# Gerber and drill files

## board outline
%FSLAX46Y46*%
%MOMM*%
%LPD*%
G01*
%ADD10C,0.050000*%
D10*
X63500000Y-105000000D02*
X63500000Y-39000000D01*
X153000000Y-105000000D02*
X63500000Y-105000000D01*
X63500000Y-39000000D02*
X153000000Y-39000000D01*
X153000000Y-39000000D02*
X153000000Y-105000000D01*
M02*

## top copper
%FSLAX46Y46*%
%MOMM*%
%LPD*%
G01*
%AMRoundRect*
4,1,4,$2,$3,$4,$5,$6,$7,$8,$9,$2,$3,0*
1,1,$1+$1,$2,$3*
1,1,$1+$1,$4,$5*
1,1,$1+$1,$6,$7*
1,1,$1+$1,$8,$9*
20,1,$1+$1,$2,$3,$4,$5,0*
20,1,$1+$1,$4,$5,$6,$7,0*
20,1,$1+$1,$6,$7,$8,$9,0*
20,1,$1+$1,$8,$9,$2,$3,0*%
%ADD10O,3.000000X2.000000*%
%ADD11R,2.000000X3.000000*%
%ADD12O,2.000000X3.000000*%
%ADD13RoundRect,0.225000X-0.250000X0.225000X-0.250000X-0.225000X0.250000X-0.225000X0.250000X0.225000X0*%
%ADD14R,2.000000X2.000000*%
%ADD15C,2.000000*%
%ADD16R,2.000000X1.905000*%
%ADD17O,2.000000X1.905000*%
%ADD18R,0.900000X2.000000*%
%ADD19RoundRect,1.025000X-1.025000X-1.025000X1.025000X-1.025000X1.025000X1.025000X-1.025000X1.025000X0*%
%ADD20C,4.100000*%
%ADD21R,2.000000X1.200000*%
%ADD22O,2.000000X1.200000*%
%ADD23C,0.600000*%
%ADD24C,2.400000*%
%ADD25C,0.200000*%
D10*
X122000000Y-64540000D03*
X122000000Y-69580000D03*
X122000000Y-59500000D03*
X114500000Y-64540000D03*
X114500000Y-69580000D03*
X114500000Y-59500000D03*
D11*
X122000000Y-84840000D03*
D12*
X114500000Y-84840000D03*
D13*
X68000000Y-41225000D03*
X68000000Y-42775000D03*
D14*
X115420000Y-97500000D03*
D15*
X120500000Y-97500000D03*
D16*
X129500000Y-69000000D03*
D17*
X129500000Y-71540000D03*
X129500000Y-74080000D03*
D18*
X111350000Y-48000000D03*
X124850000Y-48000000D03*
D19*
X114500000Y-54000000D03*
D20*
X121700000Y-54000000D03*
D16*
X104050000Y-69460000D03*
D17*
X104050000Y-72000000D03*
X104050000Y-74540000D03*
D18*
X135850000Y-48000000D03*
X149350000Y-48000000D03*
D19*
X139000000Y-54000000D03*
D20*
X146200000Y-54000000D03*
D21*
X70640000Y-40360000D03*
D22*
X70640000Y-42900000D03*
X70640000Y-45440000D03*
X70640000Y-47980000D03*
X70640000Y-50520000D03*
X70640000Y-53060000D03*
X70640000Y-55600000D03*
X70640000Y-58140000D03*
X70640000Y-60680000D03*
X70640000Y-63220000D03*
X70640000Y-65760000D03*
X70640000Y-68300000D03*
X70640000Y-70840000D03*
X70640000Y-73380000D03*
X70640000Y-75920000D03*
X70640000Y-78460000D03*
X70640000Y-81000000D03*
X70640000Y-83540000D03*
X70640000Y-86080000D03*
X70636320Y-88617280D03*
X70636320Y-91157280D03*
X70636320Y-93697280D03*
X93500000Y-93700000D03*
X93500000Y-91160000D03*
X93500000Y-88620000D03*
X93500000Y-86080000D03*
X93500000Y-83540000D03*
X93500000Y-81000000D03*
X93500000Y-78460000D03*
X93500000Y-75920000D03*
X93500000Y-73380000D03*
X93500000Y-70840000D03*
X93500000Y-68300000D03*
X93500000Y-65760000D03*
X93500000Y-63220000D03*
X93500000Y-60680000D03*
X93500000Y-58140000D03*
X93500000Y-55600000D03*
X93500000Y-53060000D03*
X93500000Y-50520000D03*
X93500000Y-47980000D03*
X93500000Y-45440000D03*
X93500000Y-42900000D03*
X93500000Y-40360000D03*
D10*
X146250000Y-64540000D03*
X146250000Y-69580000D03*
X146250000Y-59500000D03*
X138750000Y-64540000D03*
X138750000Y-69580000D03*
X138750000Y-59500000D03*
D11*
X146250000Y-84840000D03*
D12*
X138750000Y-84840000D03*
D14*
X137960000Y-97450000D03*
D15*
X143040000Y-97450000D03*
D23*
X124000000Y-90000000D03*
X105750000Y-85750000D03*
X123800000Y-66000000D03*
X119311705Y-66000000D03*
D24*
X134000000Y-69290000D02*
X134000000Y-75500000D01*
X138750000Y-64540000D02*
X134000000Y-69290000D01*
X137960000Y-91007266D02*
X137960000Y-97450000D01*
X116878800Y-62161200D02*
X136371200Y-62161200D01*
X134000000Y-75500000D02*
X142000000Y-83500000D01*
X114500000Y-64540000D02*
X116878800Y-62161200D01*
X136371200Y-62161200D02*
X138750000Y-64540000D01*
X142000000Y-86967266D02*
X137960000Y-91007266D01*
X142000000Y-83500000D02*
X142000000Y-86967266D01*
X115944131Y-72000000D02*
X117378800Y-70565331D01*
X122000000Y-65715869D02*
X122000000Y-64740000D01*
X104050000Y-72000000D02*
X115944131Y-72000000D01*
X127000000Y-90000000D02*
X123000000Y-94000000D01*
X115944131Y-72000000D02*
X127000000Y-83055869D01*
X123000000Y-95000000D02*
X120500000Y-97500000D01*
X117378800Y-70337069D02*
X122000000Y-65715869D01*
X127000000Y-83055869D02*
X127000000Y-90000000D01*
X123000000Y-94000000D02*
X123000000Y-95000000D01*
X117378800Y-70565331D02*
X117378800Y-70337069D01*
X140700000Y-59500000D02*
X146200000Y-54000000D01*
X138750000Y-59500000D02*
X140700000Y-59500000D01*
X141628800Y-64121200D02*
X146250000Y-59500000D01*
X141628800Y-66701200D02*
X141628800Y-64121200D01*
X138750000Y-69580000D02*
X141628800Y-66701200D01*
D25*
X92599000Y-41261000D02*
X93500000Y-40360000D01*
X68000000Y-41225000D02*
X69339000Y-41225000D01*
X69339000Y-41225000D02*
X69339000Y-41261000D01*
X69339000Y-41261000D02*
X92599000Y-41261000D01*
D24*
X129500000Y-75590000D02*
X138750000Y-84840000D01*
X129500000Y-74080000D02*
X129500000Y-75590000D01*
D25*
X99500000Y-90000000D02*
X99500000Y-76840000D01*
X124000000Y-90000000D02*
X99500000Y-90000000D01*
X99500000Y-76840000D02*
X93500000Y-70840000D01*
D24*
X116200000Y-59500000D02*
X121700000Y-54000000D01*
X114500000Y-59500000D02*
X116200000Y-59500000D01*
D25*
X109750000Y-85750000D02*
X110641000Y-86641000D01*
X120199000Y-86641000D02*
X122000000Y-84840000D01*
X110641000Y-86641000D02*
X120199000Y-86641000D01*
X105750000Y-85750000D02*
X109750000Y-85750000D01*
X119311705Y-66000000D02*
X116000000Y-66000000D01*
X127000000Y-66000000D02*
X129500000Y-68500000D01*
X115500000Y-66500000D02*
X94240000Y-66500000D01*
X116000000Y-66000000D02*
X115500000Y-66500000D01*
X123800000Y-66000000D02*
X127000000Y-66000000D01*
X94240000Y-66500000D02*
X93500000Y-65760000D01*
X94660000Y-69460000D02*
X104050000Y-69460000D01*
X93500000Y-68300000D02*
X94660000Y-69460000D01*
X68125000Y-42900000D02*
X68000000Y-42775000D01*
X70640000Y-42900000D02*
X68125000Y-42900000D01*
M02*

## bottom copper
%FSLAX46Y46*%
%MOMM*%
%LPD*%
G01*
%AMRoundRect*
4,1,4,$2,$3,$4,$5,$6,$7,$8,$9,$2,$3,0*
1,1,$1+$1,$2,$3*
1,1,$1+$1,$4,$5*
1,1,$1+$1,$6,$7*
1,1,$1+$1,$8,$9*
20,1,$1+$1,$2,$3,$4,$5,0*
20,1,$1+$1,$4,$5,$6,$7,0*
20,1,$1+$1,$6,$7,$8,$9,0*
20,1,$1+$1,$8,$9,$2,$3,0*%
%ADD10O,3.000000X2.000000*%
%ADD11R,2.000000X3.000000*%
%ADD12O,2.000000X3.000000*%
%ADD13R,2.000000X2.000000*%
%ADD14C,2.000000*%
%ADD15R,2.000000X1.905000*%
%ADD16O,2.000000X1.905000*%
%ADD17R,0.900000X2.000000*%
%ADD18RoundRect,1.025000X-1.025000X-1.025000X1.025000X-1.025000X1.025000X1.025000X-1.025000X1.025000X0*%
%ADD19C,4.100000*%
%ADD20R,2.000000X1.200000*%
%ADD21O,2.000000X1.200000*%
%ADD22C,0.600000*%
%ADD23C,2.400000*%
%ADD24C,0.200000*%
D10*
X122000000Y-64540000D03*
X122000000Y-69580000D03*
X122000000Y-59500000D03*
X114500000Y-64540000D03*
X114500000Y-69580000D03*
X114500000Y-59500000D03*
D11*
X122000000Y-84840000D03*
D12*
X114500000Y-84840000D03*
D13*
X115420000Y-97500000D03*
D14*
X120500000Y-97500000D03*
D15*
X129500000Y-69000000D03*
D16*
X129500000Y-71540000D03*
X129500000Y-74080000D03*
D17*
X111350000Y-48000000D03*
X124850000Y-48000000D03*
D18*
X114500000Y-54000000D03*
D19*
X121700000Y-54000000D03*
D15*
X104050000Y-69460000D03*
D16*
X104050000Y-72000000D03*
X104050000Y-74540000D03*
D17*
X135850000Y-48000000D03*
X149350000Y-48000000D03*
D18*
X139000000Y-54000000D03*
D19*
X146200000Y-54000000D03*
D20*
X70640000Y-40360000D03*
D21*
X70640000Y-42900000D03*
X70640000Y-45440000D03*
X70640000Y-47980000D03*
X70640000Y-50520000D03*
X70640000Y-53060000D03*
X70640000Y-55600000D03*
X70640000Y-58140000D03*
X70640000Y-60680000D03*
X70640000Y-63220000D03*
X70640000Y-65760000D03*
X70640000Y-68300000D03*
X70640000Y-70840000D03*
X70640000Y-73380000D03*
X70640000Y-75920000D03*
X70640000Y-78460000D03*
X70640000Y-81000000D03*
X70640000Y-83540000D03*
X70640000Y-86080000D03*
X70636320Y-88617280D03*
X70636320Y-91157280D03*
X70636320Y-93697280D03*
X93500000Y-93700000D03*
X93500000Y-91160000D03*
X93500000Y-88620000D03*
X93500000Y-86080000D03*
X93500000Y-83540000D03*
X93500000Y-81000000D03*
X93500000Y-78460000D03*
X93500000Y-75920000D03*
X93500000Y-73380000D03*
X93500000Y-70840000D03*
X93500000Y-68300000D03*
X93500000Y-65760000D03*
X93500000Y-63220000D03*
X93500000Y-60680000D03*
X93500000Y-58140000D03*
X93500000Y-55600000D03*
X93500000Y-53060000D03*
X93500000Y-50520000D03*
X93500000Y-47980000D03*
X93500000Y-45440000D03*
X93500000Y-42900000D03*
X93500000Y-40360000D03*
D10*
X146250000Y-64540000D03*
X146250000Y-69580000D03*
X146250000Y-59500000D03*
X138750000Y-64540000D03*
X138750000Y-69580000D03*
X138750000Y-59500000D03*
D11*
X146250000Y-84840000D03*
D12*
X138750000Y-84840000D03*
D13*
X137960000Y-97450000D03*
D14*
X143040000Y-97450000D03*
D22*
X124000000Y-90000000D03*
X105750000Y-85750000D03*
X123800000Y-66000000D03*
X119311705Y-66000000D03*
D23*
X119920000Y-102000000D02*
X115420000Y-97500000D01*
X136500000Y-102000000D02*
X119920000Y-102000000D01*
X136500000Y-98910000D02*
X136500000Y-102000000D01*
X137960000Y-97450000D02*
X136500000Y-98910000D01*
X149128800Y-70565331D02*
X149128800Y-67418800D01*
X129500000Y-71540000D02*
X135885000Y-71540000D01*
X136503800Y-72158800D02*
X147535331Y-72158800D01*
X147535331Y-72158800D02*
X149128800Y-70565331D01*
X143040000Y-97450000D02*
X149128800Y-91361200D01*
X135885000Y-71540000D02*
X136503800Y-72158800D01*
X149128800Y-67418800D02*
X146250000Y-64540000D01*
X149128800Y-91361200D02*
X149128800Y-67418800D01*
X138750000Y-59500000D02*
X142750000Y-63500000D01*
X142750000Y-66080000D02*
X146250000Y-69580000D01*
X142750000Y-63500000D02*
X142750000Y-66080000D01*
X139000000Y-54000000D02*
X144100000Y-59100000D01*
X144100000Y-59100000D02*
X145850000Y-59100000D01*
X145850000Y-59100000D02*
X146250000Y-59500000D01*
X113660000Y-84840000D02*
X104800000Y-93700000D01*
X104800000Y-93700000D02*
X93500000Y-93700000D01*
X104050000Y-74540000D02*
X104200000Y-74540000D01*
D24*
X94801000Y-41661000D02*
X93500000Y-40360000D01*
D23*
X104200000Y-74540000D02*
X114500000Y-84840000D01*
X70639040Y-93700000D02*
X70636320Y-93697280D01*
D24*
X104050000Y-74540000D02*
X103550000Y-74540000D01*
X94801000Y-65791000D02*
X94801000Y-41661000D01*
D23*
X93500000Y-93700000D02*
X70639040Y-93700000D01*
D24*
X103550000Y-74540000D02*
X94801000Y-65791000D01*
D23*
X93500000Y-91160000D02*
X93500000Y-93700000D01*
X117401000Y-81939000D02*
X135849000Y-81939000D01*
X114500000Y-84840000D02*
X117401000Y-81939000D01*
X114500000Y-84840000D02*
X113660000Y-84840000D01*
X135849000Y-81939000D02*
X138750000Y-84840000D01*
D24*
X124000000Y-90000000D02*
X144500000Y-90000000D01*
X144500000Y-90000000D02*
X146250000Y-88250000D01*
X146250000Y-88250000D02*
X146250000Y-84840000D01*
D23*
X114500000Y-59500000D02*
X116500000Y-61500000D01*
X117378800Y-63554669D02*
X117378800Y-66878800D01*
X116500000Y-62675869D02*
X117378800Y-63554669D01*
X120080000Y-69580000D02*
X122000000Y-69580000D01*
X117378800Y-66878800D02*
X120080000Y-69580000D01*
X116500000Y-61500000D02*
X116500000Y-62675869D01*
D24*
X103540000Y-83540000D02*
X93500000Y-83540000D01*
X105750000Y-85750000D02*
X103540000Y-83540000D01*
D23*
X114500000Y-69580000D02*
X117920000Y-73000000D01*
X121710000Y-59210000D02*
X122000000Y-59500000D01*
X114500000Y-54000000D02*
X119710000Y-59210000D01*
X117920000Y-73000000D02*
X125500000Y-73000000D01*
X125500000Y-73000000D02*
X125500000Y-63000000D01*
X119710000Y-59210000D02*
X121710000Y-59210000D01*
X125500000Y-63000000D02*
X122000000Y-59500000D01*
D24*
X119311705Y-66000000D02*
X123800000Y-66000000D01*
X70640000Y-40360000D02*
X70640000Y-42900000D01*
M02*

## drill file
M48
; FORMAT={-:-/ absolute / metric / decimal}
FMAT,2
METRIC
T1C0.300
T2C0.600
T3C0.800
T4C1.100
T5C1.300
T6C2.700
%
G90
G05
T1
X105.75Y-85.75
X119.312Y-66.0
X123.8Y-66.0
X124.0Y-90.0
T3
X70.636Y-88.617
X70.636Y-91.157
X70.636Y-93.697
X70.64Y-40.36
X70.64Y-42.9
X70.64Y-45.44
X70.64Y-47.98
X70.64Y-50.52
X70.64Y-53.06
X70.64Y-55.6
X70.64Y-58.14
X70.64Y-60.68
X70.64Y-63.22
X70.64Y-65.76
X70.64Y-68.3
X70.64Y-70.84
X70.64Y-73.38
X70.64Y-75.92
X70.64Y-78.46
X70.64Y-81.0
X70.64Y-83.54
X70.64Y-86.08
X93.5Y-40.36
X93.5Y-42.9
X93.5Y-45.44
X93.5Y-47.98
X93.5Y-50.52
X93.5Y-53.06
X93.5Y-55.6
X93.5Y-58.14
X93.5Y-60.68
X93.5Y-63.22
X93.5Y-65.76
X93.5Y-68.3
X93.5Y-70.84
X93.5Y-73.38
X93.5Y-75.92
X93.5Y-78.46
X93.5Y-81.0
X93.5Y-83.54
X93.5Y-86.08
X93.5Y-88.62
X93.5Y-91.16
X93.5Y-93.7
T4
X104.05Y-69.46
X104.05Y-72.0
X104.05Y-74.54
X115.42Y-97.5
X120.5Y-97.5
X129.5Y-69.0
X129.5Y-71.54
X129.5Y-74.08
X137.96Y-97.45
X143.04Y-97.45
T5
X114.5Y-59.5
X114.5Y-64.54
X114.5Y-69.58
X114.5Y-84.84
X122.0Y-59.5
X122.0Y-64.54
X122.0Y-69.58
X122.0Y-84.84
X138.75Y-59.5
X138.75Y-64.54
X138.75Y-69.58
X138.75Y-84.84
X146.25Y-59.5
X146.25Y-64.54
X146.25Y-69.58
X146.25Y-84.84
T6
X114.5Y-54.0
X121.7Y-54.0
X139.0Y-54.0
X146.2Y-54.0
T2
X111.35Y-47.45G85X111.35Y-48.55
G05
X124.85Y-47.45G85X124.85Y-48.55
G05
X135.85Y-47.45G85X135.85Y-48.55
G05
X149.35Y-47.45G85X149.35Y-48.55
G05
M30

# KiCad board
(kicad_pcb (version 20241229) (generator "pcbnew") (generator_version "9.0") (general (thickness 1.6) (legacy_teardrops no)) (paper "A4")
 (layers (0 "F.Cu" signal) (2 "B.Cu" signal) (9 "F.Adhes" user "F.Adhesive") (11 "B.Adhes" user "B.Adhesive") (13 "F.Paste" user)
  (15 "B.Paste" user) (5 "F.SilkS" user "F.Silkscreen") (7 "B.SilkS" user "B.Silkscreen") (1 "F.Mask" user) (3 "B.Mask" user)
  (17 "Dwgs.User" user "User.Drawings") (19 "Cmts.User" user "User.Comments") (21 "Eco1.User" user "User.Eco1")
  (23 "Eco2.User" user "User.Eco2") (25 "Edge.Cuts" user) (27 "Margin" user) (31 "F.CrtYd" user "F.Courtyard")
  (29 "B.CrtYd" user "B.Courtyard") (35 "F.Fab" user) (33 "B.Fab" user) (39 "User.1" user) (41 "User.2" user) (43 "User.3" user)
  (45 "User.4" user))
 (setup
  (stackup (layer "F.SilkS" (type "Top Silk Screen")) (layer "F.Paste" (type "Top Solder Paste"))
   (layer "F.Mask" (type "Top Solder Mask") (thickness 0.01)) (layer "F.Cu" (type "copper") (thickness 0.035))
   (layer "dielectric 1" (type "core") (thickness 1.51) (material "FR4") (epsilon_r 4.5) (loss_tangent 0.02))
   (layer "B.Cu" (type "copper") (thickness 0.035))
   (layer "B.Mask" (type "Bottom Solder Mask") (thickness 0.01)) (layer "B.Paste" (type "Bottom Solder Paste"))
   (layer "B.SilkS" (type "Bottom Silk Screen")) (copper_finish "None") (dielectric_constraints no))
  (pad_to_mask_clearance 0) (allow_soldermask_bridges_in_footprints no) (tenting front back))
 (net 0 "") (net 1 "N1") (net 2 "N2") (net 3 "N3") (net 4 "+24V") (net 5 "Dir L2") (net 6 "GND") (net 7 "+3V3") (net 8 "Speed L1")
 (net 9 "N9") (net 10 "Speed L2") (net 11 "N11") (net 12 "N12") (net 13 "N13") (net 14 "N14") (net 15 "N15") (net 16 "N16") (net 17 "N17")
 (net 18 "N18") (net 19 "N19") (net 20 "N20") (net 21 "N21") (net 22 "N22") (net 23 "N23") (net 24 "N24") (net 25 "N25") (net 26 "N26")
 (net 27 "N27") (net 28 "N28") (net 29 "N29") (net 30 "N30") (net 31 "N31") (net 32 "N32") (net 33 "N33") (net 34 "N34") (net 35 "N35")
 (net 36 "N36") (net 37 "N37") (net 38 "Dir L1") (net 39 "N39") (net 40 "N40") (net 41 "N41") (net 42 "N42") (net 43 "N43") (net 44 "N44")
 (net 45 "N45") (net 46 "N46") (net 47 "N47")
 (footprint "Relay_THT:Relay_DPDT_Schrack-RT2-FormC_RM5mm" (layer "F.Cu") (at 122 84.84 90)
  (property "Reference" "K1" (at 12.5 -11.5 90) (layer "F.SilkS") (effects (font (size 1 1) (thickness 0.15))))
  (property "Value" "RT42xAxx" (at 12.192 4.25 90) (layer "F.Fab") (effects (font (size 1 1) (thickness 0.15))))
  (pad "11" thru_hole oval (at 20.3 0 270) (size 2 3) (drill 1.3) (layers "*.Cu" "*.Mask") (remove_unused_layers no) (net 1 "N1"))
  (pad "12" thru_hole oval (at 15.26 0 270) (size 2 3) (drill 1.3) (layers "*.Cu" "*.Mask") (remove_unused_layers no) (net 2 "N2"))
  (pad "14" thru_hole oval (at 25.34 0 270) (size 2 3) (drill 1.3) (layers "*.Cu" "*.Mask") (remove_unused_layers no) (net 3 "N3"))
  (pad "21" thru_hole oval (at 20.3 -7.5 270) (size 2 3) (drill 1.3) (layers "*.Cu" "*.Mask") (remove_unused_layers no) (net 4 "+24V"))
  (pad "22" thru_hole oval (at 15.26 -7.5 270) (size 2 3) (drill 1.3) (layers "*.Cu" "*.Mask") (remove_unused_layers no) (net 3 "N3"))
  (pad "24" thru_hole oval (at 25.34 -7.5 270) (size 2 3) (drill 1.3) (layers "*.Cu" "*.Mask") (remove_unused_layers no) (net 2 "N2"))
  (pad "A1" thru_hole rect (at 0 0 270) (size 3 2) (drill 1.3) (layers "*.Cu" "*.Mask") (remove_unused_layers no) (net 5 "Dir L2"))
  (pad "A2" thru_hole oval (at 0 -7.5 270) (size 3 2) (drill 1.3) (layers "*.Cu" "*.Mask") (remove_unused_layers no) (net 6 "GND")))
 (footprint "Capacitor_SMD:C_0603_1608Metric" (layer "F.Cu") (at 68 42 -90)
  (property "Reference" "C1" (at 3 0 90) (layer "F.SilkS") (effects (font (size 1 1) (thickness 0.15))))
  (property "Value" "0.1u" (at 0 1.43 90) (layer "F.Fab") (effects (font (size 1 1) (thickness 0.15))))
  (pad "1" smd roundrect (at -0.775 0 270) (size 0.9 0.95) (layers "F.Cu" "F.Mask" "F.Paste") (roundrect_rratio 0.25) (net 6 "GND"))
  (pad "2" smd roundrect (at 0.775 0 270) (size 0.9 0.95) (layers "F.Cu" "F.Mask" "F.Paste") (roundrect_rratio 0.25) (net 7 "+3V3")))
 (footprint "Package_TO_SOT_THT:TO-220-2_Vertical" (layer "F.Cu") (at 115.42 97.5)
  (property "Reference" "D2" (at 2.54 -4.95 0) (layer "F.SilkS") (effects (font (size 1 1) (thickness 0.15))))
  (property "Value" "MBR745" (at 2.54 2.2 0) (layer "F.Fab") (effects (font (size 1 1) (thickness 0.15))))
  (pad "1" thru_hole rect (at 0 0) (size 2 2) (drill 1.1) (layers "*.Cu" "*.Mask") (remove_unused_layers no) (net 4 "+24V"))
  (pad "2" thru_hole circle (at 5.08 0) (size 2 2) (drill 1.1) (layers "*.Cu" "*.Mask") (remove_unused_layers no) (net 1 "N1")))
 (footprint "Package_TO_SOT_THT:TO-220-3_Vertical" (layer "F.Cu") (at 129.5 69 -90)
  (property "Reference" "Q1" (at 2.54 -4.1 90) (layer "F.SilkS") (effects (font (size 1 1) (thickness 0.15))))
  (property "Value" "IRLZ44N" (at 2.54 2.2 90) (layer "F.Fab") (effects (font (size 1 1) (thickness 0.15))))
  (pad "1" thru_hole rect (at 0 0 270) (size 1.905 2) (drill 1.1) (layers "*.Cu" "*.Mask") (remove_unused_layers no) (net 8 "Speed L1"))
  (pad "2" thru_hole oval (at 2.54 0 270) (size 1.905 2) (drill 1.1) (layers "*.Cu" "*.Mask") (remove_unused_layers no) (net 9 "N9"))
  (pad "3" thru_hole oval (at 5.08 0 270) (size 1.905 2) (drill 1.1) (layers "*.Cu" "*.Mask") (remove_unused_layers no) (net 6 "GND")))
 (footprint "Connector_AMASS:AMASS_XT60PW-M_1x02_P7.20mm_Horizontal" (layer "F.Cu") (at 114.5 54)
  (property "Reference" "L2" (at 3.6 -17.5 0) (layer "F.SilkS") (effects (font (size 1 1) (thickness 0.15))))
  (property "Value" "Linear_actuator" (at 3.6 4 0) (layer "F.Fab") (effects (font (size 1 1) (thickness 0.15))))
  (pad "" thru_hole rect (at -3.15 -6) (size 0.9 2) (drill oval 0.6 1.7) (layers "*.Cu" "*.Mask") (remove_unused_layers no))
  (pad "" thru_hole rect (at 10.35 -6) (size 0.9 2) (drill oval 0.6 1.7) (layers "*.Cu" "*.Mask") (remove_unused_layers no))
  (pad "1" thru_hole roundrect (at 0 0) (size 4.1 4.1) (drill 2.7) (layers "*.Cu" "*.Mask") (remove_unused_layers no)
   (roundrect_rratio 0.25) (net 3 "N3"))
  (pad "2" thru_hole circle (at 7.2 0) (size 4.1 4.1) (drill 2.7) (layers "*.Cu" "*.Mask") (remove_unused_layers no) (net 2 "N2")))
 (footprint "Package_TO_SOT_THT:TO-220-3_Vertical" (layer "F.Cu") (at 104.05 69.46 -90)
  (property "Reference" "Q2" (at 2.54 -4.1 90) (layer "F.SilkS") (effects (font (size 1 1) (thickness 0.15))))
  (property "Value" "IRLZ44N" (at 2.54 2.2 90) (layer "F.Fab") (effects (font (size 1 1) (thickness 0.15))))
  (pad "1" thru_hole rect (at 0 0 270) (size 1.905 2) (drill 1.1) (layers "*.Cu" "*.Mask") (remove_unused_layers no) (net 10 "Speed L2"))
  (pad "2" thru_hole oval (at 2.54 0 270) (size 1.905 2) (drill 1.1) (layers "*.Cu" "*.Mask") (remove_unused_layers no) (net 1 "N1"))
  (pad "3" thru_hole oval (at 5.08 0 270) (size 1.905 2) (drill 1.1) (layers "*.Cu" "*.Mask") (remove_unused_layers no) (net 6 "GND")))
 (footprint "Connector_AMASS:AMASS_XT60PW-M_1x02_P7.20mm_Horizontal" (layer "F.Cu") (at 139 54)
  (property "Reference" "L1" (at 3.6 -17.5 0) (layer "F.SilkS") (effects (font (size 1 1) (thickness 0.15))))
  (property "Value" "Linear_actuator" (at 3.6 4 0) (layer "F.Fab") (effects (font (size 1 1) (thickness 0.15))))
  (pad "" thru_hole rect (at -3.15 -6) (size 0.9 2) (drill oval 0.6 1.7) (layers "*.Cu" "*.Mask") (remove_unused_layers no))
  (pad "" thru_hole rect (at 10.35 -6) (size 0.9 2) (drill oval 0.6 1.7) (layers "*.Cu" "*.Mask") (remove_unused_layers no))
  (pad "1" thru_hole roundrect (at 0 0) (size 4.1 4.1) (drill 2.7) (layers "*.Cu" "*.Mask") (remove_unused_layers no)
   (roundrect_rratio 0.25) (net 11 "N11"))
  (pad "2" thru_hole circle (at 7.2 0) (size 4.1 4.1) (drill 2.7) (layers "*.Cu" "*.Mask") (remove_unused_layers no) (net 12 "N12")))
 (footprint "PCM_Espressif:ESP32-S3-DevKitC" (layer "F.Cu") (at 70.64 40.36)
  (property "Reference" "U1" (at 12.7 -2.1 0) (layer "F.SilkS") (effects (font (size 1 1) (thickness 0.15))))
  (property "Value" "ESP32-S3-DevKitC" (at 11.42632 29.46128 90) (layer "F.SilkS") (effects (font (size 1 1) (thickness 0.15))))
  (pad "1" thru_hole rect (at 0 0 270) (size 1.2 2) (drill 0.8) (layers "*.Cu" "*.Mask") (remove_unused_layers no) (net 7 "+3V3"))
  (pad "2" thru_hole oval (at 0 2.54 270) (size 1.2 2) (drill 0.8) (layers "*.Cu" "*.Mask") (remove_unused_layers no) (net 7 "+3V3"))
  (pad "3" thru_hole oval (at 0 5.08 270) (size 1.2 2) (drill 0.8) (layers "*.Cu" "*.Mask") (remove_unused_layers no) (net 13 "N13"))
  (pad "4" thru_hole oval (at 0 7.62 270) (size 1.2 2) (drill 0.8) (layers "*.Cu" "*.Mask") (remove_unused_layers no) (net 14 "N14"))
  (pad "5" thru_hole oval (at 0 10.16 270) (size 1.2 2) (drill 0.8) (layers "*.Cu" "*.Mask") (remove_unused_layers no) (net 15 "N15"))
  (pad "6" thru_hole oval (at 0 12.7 270) (size 1.2 2) (drill 0.8) (layers "*.Cu" "*.Mask") (remove_unused_layers no) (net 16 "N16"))
  (pad "7" thru_hole oval (at 0 15.24 270) (size 1.2 2) (drill 0.8) (layers "*.Cu" "*.Mask") (remove_unused_layers no) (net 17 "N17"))
  (pad "8" thru_hole oval (at 0 17.78 270) (size 1.2 2) (drill 0.8) (layers "*.Cu" "*.Mask") (remove_unused_layers no) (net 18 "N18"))
  (pad "9" thru_hole oval (at 0 20.32 270) (size 1.2 2) (drill 0.8) (layers "*.Cu" "*.Mask") (remove_unused_layers no) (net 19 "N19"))
  (pad "10" thru_hole oval (at 0 22.86 270) (size 1.2 2) (drill 0.8) (layers "*.Cu" "*.Mask") (remove_unused_layers no) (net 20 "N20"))
  (pad "11" thru_hole oval (at 0 25.4 270) (size 1.2 2) (drill 0.8) (layers "*.Cu" "*.Mask") (remove_unused_layers no) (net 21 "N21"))
  (pad "12" thru_hole oval (at 0 27.94 270) (size 1.2 2) (drill 0.8) (layers "*.Cu" "*.Mask") (remove_unused_layers no) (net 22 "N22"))
  (pad "13" thru_hole oval (at 0 30.48 270) (size 1.2 2) (drill 0.8) (layers "*.Cu" "*.Mask") (remove_unused_layers no) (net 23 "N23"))
  (pad "14" thru_hole oval (at 0 33.02 270) (size 1.2 2) (drill 0.8) (layers "*.Cu" "*.Mask") (remove_unused_layers no) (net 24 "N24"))
  (pad "15" thru_hole oval (at 0 35.56 270) (size 1.2 2) (drill 0.8) (layers "*.Cu" "*.Mask") (remove_unused_layers no) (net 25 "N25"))
  (pad "16" thru_hole oval (at 0 38.1 270) (size 1.2 2) (drill 0.8) (layers "*.Cu" "*.Mask") (remove_unused_layers no) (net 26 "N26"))
  (pad "17" thru_hole oval (at 0 40.64 270) (size 1.2 2) (drill 0.8) (layers "*.Cu" "*.Mask") (remove_unused_layers no) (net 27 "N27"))
  (pad "18" thru_hole oval (at 0 43.18 270) (size 1.2 2) (drill 0.8) (layers "*.Cu" "*.Mask") (remove_unused_layers no) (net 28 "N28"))
  (pad "19" thru_hole oval (at 0 45.72 270) (size 1.2 2) (drill 0.8) (layers "*.Cu" "*.Mask") (remove_unused_layers no) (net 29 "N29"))
  (pad "20" thru_hole oval (at -0.00368 48.25728 270) (size 1.2 2) (drill 0.8) (layers "*.Cu" "*.Mask") (remove_unused_layers no)
   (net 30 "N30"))
  (pad "21" thru_hole oval (at -0.00368 50.79728 270) (size 1.2 2) (drill 0.8) (layers "*.Cu" "*.Mask") (remove_unused_layers no)
   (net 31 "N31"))
  (pad "22" thru_hole oval (at -0.00368 53.33728 270) (size 1.2 2) (drill 0.8) (layers "*.Cu" "*.Mask") (remove_unused_layers no)
   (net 6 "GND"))
  (pad "23" thru_hole oval (at 22.86 53.34 270) (size 1.2 2) (drill 0.8) (layers "*.Cu" "*.Mask") (remove_unused_layers no) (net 6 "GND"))
  (pad "24" thru_hole oval (at 22.86 50.8 270) (size 1.2 2) (drill 0.8) (layers "*.Cu" "*.Mask") (remove_unused_layers no) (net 6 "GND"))
  (pad "25" thru_hole oval (at 22.86 48.26 270) (size 1.2 2) (drill 0.8) (layers "*.Cu" "*.Mask") (remove_unused_layers no) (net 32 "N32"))
  (pad "26" thru_hole oval (at 22.86 45.72 270) (size 1.2 2) (drill 0.8) (layers "*.Cu" "*.Mask") (remove_unused_layers no) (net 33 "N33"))
  (pad "27" thru_hole oval (at 22.86 43.18 270) (size 1.2 2) (drill 0.8) (layers "*.Cu" "*.Mask") (remove_unused_layers no) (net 5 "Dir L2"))
  (pad "28" thru_hole oval (at 22.86 40.64 270) (size 1.2 2) (drill 0.8) (layers "*.Cu" "*.Mask") (remove_unused_layers no) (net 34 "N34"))
  (pad "29" thru_hole oval (at 22.86 38.1 270) (size 1.2 2) (drill 0.8) (layers "*.Cu" "*.Mask") (remove_unused_layers no) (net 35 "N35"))
  (pad "30" thru_hole oval (at 22.86 35.56 270) (size 1.2 2) (drill 0.8) (layers "*.Cu" "*.Mask") (remove_unused_layers no) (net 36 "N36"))
  (pad "31" thru_hole oval (at 22.86 33.02 270) (size 1.2 2) (drill 0.8) (layers "*.Cu" "*.Mask") (remove_unused_layers no) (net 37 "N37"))
  (pad "32" thru_hole oval (at 22.86 30.48 270) (size 1.2 2) (drill 0.8) (layers "*.Cu" "*.Mask") (remove_unused_layers no)
   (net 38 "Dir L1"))
  (pad "33" thru_hole oval (at 22.86 27.94 270) (size 1.2 2) (drill 0.8) (layers "*.Cu" "*.Mask") (remove_unused_layers no)
   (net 10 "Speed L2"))
  (pad "34" thru_hole oval (at 22.86 25.4 270) (size 1.2 2) (drill 0.8) (layers "*.Cu" "*.Mask") (remove_unused_layers no)
   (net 8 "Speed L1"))
  (pad "35" thru_hole oval (at 22.86 22.86 270) (size 1.2 2) (drill 0.8) (layers "*.Cu" "*.Mask") (remove_unused_layers no) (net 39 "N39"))
  (pad "36" thru_hole oval (at 22.86 20.32 270) (size 1.2 2) (drill 0.8) (layers "*.Cu" "*.Mask") (remove_unused_layers no) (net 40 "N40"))
  (pad "37" thru_hole oval (at 22.86 17.78 270) (size 1.2 2) (drill 0.8) (layers "*.Cu" "*.Mask") (remove_unused_layers no) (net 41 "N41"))
  (pad "38" thru_hole oval (at 22.86 15.24 270) (size 1.2 2) (drill 0.8) (layers "*.Cu" "*.Mask") (remove_unused_layers no) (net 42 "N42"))
  (pad "39" thru_hole oval (at 22.86 12.7 270) (size 1.2 2) (drill 0.8) (layers "*.Cu" "*.Mask") (remove_unused_layers no) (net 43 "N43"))
  (pad "40" thru_hole oval (at 22.86 10.16 270) (size 1.2 2) (drill 0.8) (layers "*.Cu" "*.Mask") (remove_unused_layers no) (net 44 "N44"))
  (pad "41" thru_hole oval (at 22.86 7.62 270) (size 1.2 2) (drill 0.8) (layers "*.Cu" "*.Mask") (remove_unused_layers no) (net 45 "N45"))
  (pad "42" thru_hole oval (at 22.86 5.08 270) (size 1.2 2) (drill 0.8) (layers "*.Cu" "*.Mask") (remove_unused_layers no) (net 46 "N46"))
  (pad "43" thru_hole oval (at 22.86 2.54 270) (size 1.2 2) (drill 0.8) (layers "*.Cu" "*.Mask") (remove_unused_layers no) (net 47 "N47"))
  (pad "44" thru_hole oval (at 22.86 0 270) (size 1.2 2) (drill 0.8) (layers "*.Cu" "*.Mask") (remove_unused_layers no) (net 6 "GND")))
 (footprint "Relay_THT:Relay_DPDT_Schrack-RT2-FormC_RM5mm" (layer "F.Cu") (at 146.25 84.84 90)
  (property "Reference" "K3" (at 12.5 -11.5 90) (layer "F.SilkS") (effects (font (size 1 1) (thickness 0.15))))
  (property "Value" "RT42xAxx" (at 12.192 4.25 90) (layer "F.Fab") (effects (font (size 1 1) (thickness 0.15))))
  (pad "11" thru_hole oval (at 20.3 0 270) (size 2 3) (drill 1.3) (layers "*.Cu" "*.Mask") (remove_unused_layers no) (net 9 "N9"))
  (pad "12" thru_hole oval (at 15.26 0 270) (size 2 3) (drill 1.3) (layers "*.Cu" "*.Mask") (remove_unused_layers no) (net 12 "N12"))
  (pad "14" thru_hole oval (at 25.34 0 270) (size 2 3) (drill 1.3) (layers "*.Cu" "*.Mask") (remove_unused_layers no) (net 11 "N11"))
  (pad "21" thru_hole oval (at 20.3 -7.5 270) (size 2 3) (drill 1.3) (layers "*.Cu" "*.Mask") (remove_unused_layers no) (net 4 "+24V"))
  (pad "22" thru_hole oval (at 15.26 -7.5 270) (size 2 3) (drill 1.3) (layers "*.Cu" "*.Mask") (remove_unused_layers no) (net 11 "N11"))
  (pad "24" thru_hole oval (at 25.34 -7.5 270) (size 2 3) (drill 1.3) (layers "*.Cu" "*.Mask") (remove_unused_layers no) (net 12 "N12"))
  (pad "A1" thru_hole rect (at 0 0 270) (size 3 2) (drill 1.3) (layers "*.Cu" "*.Mask") (remove_unused_layers no) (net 38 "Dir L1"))
  (pad "A2" thru_hole oval (at 0 -7.5 270) (size 3 2) (drill 1.3) (layers "*.Cu" "*.Mask") (remove_unused_layers no) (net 6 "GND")))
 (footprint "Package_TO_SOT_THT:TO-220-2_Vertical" (layer "F.Cu") (at 137.96 97.45)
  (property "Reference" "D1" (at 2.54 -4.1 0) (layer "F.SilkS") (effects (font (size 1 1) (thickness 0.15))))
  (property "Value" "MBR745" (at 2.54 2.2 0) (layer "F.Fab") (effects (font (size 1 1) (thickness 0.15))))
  (pad "1" thru_hole rect (at 0 0) (size 2 2) (drill 1.1) (layers "*.Cu" "*.Mask") (remove_unused_layers no) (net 4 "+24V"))
  (pad "2" thru_hole circle (at 5.08 0) (size 2 2) (drill 1.1) (layers "*.Cu" "*.Mask") (remove_unused_layers no) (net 9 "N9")))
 (gr_line (start 63.5 105) (end 63.5 39) (stroke (width 0.05) (type default)) (layer "Edge.Cuts"))
 (gr_line (start 153 105) (end 63.5 105) (stroke (width 0.05) (type default)) (layer "Edge.Cuts"))
 (gr_line (start 63.5 39) (end 153 39) (stroke (width 0.05) (type default)) (layer "Edge.Cuts"))
 (gr_line (start 153 39) (end 153 105) (stroke (width 0.05) (type default)) (layer "Edge.Cuts"))
 (segment (start 134 69.29) (end 134 75.5) (width 2.4) (layer "F.Cu") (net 4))
 (segment (start 138.75 64.54) (end 134 69.29) (width 2.4) (layer "F.Cu") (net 4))
 (segment (start 137.96 91.007266) (end 137.96 97.45) (width 2.4) (layer "F.Cu") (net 4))
 (segment (start 116.8788 62.1612) (end 136.3712 62.1612) (width 2.4) (layer "F.Cu") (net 4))
 (segment (start 134 75.5) (end 142 83.5) (width 2.4) (layer "F.Cu") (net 4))
 (segment (start 114.5 64.54) (end 116.8788 62.1612) (width 2.4) (layer "F.Cu") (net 4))
 (segment (start 136.3712 62.1612) (end 138.75 64.54) (width 2.4) (layer "F.Cu") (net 4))
 (segment (start 142 86.967266) (end 137.96 91.007266) (width 2.4) (layer "F.Cu") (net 4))
 (segment (start 142 83.5) (end 142 86.967266) (width 2.4) (layer "F.Cu") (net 4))
 (segment (start 119.92 102) (end 115.42 97.5) (width 2.4) (layer "B.Cu") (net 4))
 (segment (start 136.5 102) (end 119.92 102) (width 2.4) (layer "B.Cu") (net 4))
 (segment (start 136.5 98.91) (end 136.5 102) (width 2.4) (layer "B.Cu") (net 4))
 (segment (start 137.96 97.45) (end 136.5 98.91) (width 2.4) (layer "B.Cu") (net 4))
 (segment (start 149.1288 70.565331) (end 149.1288 67.4188) (width 2.4) (layer "B.Cu") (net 9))
 (segment (start 129.5 71.54) (end 135.885 71.54) (width 2.4) (layer "B.Cu") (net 9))
 (segment (start 136.5038 72.1588) (end 147.535331 72.1588) (width 2.4) (layer "B.Cu") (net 9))
 (segment (start 147.535331 72.1588) (end 149.1288 70.565331) (width 2.4) (layer "B.Cu") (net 9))
 (segment (start 143.04 97.45) (end 149.1288 91.3612) (width 2.4) (layer "B.Cu") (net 9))
 (segment (start 135.885 71.54) (end 136.5038 72.1588) (width 2.4) (layer "B.Cu") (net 9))
 (segment (start 149.1288 67.4188) (end 146.25 64.54) (width 2.4) (layer "B.Cu") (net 9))
 (segment (start 149.1288 91.3612) (end 149.1288 67.4188) (width 2.4) (layer "B.Cu") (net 9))
 (segment (start 115.944131 72) (end 117.3788 70.565331) (width 2.4) (layer "F.Cu") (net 1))
 (segment (start 122 65.715869) (end 122 64.74) (width 2.4) (layer "F.Cu") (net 1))
 (segment (start 104.05 72) (end 115.944131 72) (width 2.4) (layer "F.Cu") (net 1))
 (segment (start 127 90) (end 123 94) (width 2.4) (layer "F.Cu") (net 1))
 (segment (start 115.944131 72) (end 127 83.055869) (width 2.4) (layer "F.Cu") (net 1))
 (segment (start 123 95) (end 120.5 97.5) (width 2.4) (layer "F.Cu") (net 1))
 (segment (start 117.3788 70.337069) (end 122 65.715869) (width 2.4) (layer "F.Cu") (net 1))
 (segment (start 127 83.055869) (end 127 90) (width 2.4) (layer "F.Cu") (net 1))
 (segment (start 123 94) (end 123 95) (width 2.4) (layer "F.Cu") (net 1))
 (segment (start 117.3788 70.565331) (end 117.3788 70.337069) (width 2.4) (layer "F.Cu") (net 1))
 (segment (start 140.7 59.5) (end 146.2 54) (width 2.4) (layer "F.Cu") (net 12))
 (segment (start 138.75 59.5) (end 140.7 59.5) (width 2.4) (layer "F.Cu") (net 12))
 (segment (start 138.75 59.5) (end 142.75 63.5) (width 2.4) (layer "B.Cu") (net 12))
 (segment (start 142.75 66.08) (end 146.25 69.58) (width 2.4) (layer "B.Cu") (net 12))
 (segment (start 142.75 63.5) (end 142.75 66.08) (width 2.4) (layer "B.Cu") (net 12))
 (segment (start 141.6288 64.1212) (end 146.25 59.5) (width 2.4) (layer "F.Cu") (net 11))
 (segment (start 141.6288 66.7012) (end 141.6288 64.1212) (width 2.4) (layer "F.Cu") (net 11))
 (segment (start 138.75 69.58) (end 141.6288 66.7012) (width 2.4) (layer "F.Cu") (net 11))
 (segment (start 139 54) (end 144.1 59.1) (width 2.4) (layer "B.Cu") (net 11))
 (segment (start 144.1 59.1) (end 145.85 59.1) (width 2.4) (layer "B.Cu") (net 11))
 (segment (start 145.85 59.1) (end 146.25 59.5) (width 2.4) (layer "B.Cu") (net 11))
 (segment (start 92.599 41.261) (end 93.5 40.36) (width 0.2) (layer "F.Cu") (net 6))
 (segment (start 68 41.225) (end 69.339 41.225) (width 0.2) (layer "F.Cu") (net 6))
 (segment (start 69.339 41.225) (end 69.339 41.261) (width 0.2) (layer "F.Cu") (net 6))
 (segment (start 69.339 41.261) (end 92.599 41.261) (width 0.2) (layer "F.Cu") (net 6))
 (segment (start 129.5 75.59) (end 138.75 84.84) (width 2.4) (layer "F.Cu") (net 6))
 (segment (start 129.5 74.08) (end 129.5 75.59) (width 2.4) (layer "F.Cu") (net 6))
 (segment (start 113.66 84.84) (end 104.8 93.7) (width 2.4) (layer "B.Cu") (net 6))
 (segment (start 104.8 93.7) (end 93.5 93.7) (width 2.4) (layer "B.Cu") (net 6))
 (segment (start 104.05 74.54) (end 104.2 74.54) (width 2.4) (layer "B.Cu") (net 6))
 (segment (start 94.801 41.661) (end 93.5 40.36) (width 0.2) (layer "B.Cu") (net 6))
 (segment (start 104.2 74.54) (end 114.5 84.84) (width 2.4) (layer "B.Cu") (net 6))
 (segment (start 70.63904 93.7) (end 70.63632 93.69728) (width 2.4) (layer "B.Cu") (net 6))
 (segment (start 104.05 74.54) (end 103.55 74.54) (width 0.2) (layer "B.Cu") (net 6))
 (segment (start 94.801 65.791) (end 94.801 41.661) (width 0.2) (layer "B.Cu") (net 6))
 (segment (start 93.5 93.7) (end 70.63904 93.7) (width 2.4) (layer "B.Cu") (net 6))
 (segment (start 103.55 74.54) (end 94.801 65.791) (width 0.2) (layer "B.Cu") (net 6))
 (segment (start 93.5 91.16) (end 93.5 93.7) (width 2.4) (layer "B.Cu") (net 6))
 (segment (start 117.401 81.939) (end 135.849 81.939) (width 2.4) (layer "B.Cu") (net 6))
 (segment (start 114.5 84.84) (end 117.401 81.939) (width 2.4) (layer "B.Cu") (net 6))
 (segment (start 114.5 84.84) (end 113.66 84.84) (width 2.4) (layer "B.Cu") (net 6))
 (segment (start 135.849 81.939) (end 138.75 84.84) (width 2.4) (layer "B.Cu") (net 6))
 (segment (start 99.5 90) (end 99.5 76.84) (width 0.2) (layer "F.Cu") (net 38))
 (segment (start 124 90) (end 99.5 90) (width 0.2) (layer "F.Cu") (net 38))
 (segment (start 99.5 76.84) (end 93.5 70.84) (width 0.2) (layer "F.Cu") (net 38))
 (via (at 124 90) (size 0.6) (drill 0.3) (layers "F.Cu" "B.Cu") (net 38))
 (segment (start 124 90) (end 144.5 90) (width 0.2) (layer "B.Cu") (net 38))
 (segment (start 144.5 90) (end 146.25 88.25) (width 0.2) (layer "B.Cu") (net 38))
 (segment (start 146.25 88.25) (end 146.25 84.84) (width 0.2) (layer "B.Cu") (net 38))
 (segment (start 116.2 59.5) (end 121.7 54) (width 2.4) (layer "F.Cu") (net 2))
 (segment (start 114.5 59.5) (end 116.2 59.5) (width 2.4) (layer "F.Cu") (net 2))
 (segment (start 114.5 59.5) (end 116.5 61.5) (width 2.4) (layer "B.Cu") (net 2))
 (segment (start 117.3788 63.554669) (end 117.3788 66.8788) (width 2.4) (layer "B.Cu") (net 2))
 (segment (start 116.5 62.675869) (end 117.3788 63.554669) (width 2.4) (layer "B.Cu") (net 2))
 (segment (start 120.08 69.58) (end 122 69.58) (width 2.4) (layer "B.Cu") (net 2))
 (segment (start 117.3788 66.8788) (end 120.08 69.58) (width 2.4) (layer "B.Cu") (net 2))
 (segment (start 116.5 61.5) (end 116.5 62.675869) (width 2.4) (layer "B.Cu") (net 2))
 (segment (start 109.75 85.75) (end 110.641 86.641) (width 0.2) (layer "F.Cu") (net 5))
 (segment (start 120.199 86.641) (end 122 84.84) (width 0.2) (layer "F.Cu") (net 5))
 (segment (start 110.641 86.641) (end 120.199 86.641) (width 0.2) (layer "F.Cu") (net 5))
 (segment (start 105.75 85.75) (end 109.75 85.75) (width 0.2) (layer "F.Cu") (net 5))
 (via (at 105.75 85.75) (size 0.6) (drill 0.3) (layers "F.Cu" "B.Cu") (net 5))
 (segment (start 103.54 83.54) (end 93.5 83.54) (width 0.2) (layer "B.Cu") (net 5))
 (segment (start 105.75 85.75) (end 103.54 83.54) (width 0.2) (layer "B.Cu") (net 5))
 (segment (start 114.5 69.58) (end 117.92 73) (width 2.4) (layer "B.Cu") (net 3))
 (segment (start 121.71 59.21) (end 122 59.5) (width 2.4) (layer "B.Cu") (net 3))
 (segment (start 114.5 54) (end 119.71 59.21) (width 2.4) (layer "B.Cu") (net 3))
 (segment (start 117.92 73) (end 125.5 73) (width 2.4) (layer "B.Cu") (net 3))
 (segment (start 125.5 73) (end 125.5 63) (width 2.4) (layer "B.Cu") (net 3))
 (segment (start 119.71 59.21) (end 121.71 59.21) (width 2.4) (layer "B.Cu") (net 3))
 (segment (start 125.5 63) (end 122 59.5) (width 2.4) (layer "B.Cu") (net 3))
 (segment (start 119.311705 66) (end 116 66) (width 0.2) (layer "F.Cu") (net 8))
 (segment (start 127 66) (end 129.5 68.5) (width 0.2) (layer "F.Cu") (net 8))
 (segment (start 115.5 66.5) (end 94.24 66.5) (width 0.2) (layer "F.Cu") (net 8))
 (segment (start 116 66) (end 115.5 66.5) (width 0.2) (layer "F.Cu") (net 8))
 (segment (start 123.8 66) (end 127 66) (width 0.2) (layer "F.Cu") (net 8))
 (segment (start 94.24 66.5) (end 93.5 65.76) (width 0.2) (layer "F.Cu") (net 8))
 (via (at 123.8 66) (size 0.6) (drill 0.3) (layers "F.Cu" "B.Cu") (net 8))
 (via (at 119.311705 66) (size 0.6) (drill 0.3) (layers "F.Cu" "B.Cu") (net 8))
 (segment (start 119.311705 66) (end 123.8 66) (width 0.2) (layer "B.Cu") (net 8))
 (segment (start 94.66 69.46) (end 104.05 69.46) (width 0.2) (layer "F.Cu") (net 10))
 (segment (start 93.5 68.3) (end 94.66 69.46) (width 0.2) (layer "F.Cu") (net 10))
 (segment (start 68.125 42.9) (end 68 42.775) (width 0.2) (layer "F.Cu") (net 7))
 (segment (start 70.64 42.9) (end 68.125 42.9) (width 0.2) (layer "F.Cu") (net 7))
 (segment (start 70.64 40.36) (end 70.64 42.9) (width 0.2) (layer "B.Cu") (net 7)))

